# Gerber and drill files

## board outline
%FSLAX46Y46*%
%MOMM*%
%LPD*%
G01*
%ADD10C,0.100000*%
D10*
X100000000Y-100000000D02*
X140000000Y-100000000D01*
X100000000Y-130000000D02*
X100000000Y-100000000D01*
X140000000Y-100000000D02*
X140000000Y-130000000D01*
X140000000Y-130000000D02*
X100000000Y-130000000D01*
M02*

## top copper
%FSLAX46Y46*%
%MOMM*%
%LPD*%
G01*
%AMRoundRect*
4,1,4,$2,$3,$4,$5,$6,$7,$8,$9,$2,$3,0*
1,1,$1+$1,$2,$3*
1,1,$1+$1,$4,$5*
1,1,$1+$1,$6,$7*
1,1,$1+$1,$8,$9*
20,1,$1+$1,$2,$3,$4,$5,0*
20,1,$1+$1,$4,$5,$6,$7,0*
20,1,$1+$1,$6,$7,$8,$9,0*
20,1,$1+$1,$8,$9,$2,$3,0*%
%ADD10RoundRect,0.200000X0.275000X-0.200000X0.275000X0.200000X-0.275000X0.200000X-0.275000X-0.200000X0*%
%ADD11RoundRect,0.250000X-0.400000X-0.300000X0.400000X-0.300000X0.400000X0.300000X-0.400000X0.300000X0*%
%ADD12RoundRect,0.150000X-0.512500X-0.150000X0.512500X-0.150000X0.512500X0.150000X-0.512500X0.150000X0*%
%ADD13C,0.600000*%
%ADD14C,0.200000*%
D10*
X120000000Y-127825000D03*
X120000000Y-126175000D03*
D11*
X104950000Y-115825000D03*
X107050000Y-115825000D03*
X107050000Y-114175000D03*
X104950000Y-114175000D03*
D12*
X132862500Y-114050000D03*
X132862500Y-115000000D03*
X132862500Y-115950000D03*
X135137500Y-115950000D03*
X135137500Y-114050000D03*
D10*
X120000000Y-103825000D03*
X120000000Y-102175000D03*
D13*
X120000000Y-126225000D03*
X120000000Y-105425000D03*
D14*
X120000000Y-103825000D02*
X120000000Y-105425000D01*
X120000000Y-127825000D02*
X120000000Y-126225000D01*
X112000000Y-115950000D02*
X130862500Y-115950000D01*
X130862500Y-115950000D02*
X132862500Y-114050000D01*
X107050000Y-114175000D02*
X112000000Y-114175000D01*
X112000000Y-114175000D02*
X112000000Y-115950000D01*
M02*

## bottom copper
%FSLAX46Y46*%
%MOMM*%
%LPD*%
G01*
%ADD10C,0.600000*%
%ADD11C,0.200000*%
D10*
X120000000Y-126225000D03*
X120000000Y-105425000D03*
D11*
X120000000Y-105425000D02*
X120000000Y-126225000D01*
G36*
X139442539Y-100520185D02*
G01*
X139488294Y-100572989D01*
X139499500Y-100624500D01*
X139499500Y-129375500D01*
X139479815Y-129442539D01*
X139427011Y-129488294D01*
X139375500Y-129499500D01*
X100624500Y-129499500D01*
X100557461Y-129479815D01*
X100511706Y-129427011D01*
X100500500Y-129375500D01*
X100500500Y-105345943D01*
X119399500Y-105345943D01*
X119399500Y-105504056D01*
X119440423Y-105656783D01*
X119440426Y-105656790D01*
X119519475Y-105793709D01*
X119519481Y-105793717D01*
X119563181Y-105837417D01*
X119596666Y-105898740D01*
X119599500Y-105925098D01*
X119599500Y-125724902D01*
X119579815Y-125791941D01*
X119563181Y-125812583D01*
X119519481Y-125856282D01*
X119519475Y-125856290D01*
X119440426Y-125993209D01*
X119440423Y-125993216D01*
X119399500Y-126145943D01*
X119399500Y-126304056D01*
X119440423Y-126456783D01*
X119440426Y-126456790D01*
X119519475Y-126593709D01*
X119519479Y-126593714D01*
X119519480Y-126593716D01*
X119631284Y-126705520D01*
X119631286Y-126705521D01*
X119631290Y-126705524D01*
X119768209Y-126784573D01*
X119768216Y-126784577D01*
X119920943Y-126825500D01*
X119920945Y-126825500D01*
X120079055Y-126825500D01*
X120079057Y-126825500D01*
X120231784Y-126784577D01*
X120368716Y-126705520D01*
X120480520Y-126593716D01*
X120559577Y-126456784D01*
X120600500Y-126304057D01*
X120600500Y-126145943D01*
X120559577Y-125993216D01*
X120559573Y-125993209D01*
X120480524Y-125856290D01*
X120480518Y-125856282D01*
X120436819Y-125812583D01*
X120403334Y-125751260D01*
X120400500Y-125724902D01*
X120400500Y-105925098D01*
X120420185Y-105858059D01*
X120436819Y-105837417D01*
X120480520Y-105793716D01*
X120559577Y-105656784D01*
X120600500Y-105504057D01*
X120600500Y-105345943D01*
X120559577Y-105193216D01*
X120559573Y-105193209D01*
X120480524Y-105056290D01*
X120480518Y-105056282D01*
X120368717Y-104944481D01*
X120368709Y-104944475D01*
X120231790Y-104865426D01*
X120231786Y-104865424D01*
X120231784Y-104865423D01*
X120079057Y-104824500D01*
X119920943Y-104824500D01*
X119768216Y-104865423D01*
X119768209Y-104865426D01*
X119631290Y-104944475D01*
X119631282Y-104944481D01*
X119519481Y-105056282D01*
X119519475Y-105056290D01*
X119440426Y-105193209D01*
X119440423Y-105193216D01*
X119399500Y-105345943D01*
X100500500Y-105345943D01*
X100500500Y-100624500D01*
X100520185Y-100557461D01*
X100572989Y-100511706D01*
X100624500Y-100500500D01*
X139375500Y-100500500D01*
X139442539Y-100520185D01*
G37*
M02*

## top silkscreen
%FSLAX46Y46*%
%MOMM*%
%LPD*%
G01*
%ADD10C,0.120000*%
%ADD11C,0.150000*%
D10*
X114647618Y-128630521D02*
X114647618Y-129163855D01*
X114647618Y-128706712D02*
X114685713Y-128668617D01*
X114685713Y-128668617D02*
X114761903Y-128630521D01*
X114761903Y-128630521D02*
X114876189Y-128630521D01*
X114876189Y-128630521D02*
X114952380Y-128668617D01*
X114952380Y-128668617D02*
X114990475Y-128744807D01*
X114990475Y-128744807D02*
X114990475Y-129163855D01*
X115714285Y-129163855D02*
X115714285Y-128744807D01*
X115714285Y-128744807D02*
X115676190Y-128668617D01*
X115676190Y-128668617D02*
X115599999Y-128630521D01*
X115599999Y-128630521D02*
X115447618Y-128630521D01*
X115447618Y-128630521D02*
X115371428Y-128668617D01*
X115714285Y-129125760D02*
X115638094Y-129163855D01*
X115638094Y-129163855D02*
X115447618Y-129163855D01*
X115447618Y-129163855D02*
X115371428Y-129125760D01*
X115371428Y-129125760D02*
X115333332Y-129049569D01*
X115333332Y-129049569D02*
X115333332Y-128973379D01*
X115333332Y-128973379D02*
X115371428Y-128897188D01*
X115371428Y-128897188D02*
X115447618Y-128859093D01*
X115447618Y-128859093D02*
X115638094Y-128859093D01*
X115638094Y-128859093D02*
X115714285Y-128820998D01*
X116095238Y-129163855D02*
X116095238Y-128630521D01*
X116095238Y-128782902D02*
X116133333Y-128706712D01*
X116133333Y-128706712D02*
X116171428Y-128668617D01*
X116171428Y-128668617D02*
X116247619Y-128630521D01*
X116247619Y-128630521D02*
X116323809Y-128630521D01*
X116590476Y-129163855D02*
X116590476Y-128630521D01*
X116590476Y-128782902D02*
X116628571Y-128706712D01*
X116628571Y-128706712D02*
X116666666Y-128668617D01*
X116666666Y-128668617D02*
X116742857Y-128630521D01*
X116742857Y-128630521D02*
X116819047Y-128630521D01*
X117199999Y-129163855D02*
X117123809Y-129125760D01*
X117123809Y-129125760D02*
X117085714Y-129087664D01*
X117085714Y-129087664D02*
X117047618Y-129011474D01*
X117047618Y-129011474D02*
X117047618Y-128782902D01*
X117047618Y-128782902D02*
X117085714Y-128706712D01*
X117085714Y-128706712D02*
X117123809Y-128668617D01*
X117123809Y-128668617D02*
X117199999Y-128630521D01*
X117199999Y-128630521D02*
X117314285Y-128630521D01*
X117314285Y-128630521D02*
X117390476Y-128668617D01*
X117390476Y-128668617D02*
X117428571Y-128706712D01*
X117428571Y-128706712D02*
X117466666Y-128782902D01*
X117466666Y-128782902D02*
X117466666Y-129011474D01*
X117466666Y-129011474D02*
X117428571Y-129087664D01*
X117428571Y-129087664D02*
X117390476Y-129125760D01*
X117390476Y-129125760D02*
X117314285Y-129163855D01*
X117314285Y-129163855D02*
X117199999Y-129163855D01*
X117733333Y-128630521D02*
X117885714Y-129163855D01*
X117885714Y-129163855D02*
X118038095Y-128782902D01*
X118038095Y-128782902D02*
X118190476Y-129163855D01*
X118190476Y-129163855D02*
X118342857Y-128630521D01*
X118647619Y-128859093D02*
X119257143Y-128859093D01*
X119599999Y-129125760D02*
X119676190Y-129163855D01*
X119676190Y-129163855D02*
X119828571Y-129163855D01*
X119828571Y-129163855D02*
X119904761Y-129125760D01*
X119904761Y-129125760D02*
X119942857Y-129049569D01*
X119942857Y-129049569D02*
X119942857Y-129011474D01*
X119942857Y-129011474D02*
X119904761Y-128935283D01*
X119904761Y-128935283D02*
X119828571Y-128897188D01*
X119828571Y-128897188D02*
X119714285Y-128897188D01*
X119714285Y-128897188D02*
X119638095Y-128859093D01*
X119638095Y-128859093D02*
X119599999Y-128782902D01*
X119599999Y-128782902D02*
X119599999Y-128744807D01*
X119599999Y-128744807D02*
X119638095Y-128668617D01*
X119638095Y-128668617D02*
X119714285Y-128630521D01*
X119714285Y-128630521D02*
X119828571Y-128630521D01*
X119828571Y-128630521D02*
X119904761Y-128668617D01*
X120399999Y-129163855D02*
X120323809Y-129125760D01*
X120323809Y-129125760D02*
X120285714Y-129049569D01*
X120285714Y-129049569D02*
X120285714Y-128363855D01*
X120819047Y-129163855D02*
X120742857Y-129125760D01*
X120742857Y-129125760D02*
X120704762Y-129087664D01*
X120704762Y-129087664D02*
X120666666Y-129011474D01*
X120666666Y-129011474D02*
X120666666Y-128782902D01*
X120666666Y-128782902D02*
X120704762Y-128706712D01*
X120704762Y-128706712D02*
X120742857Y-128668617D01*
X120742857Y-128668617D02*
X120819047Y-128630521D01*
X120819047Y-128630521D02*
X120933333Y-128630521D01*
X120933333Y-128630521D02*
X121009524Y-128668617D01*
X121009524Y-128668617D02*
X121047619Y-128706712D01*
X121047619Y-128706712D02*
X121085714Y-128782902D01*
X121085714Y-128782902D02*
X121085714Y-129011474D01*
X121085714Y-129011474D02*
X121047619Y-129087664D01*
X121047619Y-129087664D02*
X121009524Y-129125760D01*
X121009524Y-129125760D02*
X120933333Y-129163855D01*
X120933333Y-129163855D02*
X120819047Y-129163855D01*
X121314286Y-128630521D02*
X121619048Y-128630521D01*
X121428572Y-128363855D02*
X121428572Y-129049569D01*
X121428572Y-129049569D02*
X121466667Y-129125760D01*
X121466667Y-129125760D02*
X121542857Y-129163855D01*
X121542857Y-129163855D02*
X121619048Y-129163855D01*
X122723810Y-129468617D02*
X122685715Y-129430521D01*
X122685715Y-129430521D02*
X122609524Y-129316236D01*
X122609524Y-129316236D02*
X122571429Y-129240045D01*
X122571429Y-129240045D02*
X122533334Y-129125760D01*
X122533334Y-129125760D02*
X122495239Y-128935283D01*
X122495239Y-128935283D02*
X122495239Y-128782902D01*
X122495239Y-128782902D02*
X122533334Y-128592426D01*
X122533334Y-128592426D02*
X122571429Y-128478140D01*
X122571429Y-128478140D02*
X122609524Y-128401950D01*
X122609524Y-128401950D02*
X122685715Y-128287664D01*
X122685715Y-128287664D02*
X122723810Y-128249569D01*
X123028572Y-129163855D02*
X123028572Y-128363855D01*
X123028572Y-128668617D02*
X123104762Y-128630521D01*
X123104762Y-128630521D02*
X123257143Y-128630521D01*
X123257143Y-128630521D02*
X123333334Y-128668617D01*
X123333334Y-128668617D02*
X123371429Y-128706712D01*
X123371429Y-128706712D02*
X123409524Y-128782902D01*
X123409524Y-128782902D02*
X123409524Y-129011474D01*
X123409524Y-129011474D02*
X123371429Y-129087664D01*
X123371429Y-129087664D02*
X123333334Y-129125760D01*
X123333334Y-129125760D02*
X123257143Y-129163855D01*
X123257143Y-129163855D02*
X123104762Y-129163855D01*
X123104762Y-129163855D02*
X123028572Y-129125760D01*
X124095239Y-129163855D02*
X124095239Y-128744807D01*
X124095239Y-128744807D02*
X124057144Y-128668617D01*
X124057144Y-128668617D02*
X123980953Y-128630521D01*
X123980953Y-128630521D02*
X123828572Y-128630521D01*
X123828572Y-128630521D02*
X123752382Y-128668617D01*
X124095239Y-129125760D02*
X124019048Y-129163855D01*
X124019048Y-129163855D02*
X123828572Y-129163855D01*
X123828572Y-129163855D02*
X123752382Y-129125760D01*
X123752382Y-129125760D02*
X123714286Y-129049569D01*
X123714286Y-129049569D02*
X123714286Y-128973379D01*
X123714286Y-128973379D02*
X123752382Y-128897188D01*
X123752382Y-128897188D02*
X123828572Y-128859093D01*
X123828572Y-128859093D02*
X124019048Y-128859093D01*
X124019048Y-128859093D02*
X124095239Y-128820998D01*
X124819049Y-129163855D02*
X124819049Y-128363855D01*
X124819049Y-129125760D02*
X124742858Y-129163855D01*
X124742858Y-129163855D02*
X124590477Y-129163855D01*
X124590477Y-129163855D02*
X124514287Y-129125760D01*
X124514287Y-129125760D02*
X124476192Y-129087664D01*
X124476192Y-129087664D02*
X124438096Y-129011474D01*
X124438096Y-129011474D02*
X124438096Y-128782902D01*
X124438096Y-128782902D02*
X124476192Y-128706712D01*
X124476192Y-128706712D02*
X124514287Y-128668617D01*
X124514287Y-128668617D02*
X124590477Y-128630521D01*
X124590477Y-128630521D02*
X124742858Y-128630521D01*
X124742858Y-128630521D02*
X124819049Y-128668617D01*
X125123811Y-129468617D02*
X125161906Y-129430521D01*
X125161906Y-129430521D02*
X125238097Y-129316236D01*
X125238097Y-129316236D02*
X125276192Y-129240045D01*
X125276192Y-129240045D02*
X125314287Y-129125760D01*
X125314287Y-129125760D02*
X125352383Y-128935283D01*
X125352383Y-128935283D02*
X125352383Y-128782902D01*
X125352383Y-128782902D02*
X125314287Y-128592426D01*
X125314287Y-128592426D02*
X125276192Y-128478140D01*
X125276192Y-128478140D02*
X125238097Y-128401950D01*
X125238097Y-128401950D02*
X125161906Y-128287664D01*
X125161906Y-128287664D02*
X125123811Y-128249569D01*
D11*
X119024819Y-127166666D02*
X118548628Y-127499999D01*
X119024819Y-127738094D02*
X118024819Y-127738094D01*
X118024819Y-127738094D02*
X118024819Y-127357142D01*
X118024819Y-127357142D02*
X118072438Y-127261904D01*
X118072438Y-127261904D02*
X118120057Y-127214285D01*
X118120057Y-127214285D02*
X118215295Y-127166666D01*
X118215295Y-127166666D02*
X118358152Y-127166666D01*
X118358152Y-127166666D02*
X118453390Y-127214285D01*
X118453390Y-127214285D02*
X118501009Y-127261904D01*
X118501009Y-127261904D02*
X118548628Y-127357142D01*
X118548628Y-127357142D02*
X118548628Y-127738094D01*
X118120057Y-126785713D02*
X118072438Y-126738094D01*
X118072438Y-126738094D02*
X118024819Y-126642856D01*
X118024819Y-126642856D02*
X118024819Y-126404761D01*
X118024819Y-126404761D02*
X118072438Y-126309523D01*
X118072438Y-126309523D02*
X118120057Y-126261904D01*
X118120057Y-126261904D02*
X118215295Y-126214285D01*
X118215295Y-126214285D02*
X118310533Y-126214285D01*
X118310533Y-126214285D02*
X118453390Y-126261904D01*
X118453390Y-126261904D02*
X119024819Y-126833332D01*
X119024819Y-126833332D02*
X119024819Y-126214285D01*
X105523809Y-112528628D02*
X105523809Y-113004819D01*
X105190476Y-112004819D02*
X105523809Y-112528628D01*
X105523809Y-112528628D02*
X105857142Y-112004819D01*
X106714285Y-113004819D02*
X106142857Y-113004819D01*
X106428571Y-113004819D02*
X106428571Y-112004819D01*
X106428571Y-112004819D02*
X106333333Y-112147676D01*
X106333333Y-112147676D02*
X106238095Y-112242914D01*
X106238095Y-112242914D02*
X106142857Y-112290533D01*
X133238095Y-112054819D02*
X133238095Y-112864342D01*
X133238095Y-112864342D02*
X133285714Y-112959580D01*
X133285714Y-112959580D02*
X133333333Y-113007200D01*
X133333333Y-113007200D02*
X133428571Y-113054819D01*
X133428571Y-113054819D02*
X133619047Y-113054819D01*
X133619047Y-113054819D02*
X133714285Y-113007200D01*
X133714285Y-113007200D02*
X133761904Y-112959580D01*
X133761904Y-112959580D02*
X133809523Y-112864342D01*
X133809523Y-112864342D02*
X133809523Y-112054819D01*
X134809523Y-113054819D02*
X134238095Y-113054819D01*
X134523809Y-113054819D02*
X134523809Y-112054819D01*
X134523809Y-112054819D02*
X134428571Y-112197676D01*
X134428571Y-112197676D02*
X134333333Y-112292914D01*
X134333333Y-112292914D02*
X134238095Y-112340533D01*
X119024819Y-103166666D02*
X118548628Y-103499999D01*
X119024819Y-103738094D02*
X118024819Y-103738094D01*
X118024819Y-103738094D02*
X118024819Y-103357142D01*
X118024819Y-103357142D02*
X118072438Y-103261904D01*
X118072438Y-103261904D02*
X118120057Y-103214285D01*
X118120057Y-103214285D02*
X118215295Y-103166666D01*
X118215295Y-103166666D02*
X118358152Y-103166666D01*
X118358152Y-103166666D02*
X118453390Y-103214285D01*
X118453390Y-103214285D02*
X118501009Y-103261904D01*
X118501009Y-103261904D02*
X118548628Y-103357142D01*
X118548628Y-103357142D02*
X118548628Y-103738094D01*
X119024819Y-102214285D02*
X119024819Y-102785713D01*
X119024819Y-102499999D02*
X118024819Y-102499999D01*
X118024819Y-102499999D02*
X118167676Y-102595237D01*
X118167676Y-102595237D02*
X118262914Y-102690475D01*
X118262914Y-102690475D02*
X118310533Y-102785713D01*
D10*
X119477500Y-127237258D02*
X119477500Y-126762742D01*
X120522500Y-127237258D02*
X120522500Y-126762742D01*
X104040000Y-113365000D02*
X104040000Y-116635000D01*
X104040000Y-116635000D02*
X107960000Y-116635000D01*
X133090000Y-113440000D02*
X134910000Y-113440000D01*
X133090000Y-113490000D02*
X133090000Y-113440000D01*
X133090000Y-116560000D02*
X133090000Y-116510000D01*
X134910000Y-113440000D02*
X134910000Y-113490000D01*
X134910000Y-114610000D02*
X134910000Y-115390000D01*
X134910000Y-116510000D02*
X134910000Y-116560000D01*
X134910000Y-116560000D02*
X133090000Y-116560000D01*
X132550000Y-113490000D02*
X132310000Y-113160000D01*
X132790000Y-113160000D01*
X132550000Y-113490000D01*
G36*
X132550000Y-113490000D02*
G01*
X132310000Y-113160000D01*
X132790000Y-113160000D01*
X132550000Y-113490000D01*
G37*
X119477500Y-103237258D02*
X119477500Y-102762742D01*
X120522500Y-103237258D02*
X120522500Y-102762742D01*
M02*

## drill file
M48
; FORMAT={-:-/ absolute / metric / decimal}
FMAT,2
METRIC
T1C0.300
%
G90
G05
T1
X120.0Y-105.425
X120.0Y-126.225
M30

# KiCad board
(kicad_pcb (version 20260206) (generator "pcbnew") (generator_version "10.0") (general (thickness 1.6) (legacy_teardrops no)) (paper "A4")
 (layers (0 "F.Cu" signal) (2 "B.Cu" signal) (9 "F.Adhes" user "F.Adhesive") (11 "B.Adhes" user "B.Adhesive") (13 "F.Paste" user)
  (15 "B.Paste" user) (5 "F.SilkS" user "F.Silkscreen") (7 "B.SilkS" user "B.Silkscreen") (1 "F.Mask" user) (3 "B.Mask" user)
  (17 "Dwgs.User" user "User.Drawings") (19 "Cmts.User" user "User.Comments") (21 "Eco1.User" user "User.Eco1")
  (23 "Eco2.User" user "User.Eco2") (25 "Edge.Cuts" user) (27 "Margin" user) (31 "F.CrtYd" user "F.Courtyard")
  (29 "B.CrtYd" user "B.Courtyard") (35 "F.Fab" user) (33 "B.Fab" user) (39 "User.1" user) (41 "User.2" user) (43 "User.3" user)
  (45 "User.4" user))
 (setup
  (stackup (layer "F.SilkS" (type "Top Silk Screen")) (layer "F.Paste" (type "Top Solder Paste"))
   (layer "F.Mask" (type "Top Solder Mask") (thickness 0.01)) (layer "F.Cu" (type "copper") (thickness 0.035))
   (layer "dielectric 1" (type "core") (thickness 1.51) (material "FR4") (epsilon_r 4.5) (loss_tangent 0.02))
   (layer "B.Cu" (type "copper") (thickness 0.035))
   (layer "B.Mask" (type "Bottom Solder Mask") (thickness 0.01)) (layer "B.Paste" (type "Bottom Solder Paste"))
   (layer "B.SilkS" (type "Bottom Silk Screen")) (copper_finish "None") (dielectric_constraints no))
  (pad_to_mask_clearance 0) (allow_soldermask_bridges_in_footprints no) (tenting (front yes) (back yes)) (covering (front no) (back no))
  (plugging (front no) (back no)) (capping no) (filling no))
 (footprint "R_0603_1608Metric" (layer "F.Cu") (at 120 127 90)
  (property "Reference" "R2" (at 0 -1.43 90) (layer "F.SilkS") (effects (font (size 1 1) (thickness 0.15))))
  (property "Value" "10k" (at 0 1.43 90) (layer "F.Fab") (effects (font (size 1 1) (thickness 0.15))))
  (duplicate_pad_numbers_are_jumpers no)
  (fp_line (start -0.237258 -0.5225) (end 0.237258 -0.5225) (stroke (width 0.12) (type solid)) (layer "F.SilkS"))
  (fp_line (start -0.237258 0.5225) (end 0.237258 0.5225) (stroke (width 0.12) (type solid)) (layer "F.SilkS"))
  (pad "1" smd roundrect (at -0.825 0 90) (size 0.8 0.95) (layers "F.Cu" "F.Mask" "F.Paste") (roundrect_rratio 0.25) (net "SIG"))
  (pad "2" smd roundrect (at 0.825 0 90) (size 0.8 0.95) (layers "F.Cu" "F.Mask" "F.Paste") (roundrect_rratio 0.25) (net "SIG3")))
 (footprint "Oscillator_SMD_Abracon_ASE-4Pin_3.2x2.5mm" (layer "F.Cu") (at 106 115)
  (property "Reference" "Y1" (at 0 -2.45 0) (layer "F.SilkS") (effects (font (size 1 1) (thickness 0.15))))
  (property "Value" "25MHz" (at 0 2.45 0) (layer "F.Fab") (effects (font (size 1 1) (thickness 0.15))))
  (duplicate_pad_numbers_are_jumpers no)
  (fp_line (start -1.96 -1.635) (end -1.96 1.635) (stroke (width 0.12) (type solid)) (layer "F.SilkS"))
  (fp_line (start -1.96 1.635) (end 1.96 1.635) (stroke (width 0.12) (type solid)) (layer "F.SilkS"))
  (pad "1" smd roundrect (at -1.05 0.825) (size 1.3 1.1) (layers "F.Cu" "F.Mask" "F.Paste") (roundrect_rratio 0.227273) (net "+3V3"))
  (pad "2" smd roundrect (at 1.05 0.825) (size 1.3 1.1) (layers "F.Cu" "F.Mask" "F.Paste") (roundrect_rratio 0.227273) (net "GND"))
  (pad "3" smd roundrect (at 1.05 -0.825) (size 1.3 1.1) (layers "F.Cu" "F.Mask" "F.Paste") (roundrect_rratio 0.227273) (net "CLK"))
  (pad "4" smd roundrect (at -1.05 -0.825) (size 1.3 1.1) (layers "F.Cu" "F.Mask" "F.Paste") (roundrect_rratio 0.227273) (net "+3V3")))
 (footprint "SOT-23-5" (layer "F.Cu") (at 134 115)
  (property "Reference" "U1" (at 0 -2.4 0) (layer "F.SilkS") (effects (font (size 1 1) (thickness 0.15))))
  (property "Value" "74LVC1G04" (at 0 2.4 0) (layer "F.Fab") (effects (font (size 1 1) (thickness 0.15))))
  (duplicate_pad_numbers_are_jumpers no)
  (fp_line (start -0.91 -1.56) (end 0.91 -1.56) (stroke (width 0.12) (type solid)) (layer "F.SilkS"))
  (fp_line (start -0.91 -1.51) (end -0.91 -1.56) (stroke (width 0.12) (type solid)) (layer "F.SilkS"))
  (fp_line (start -0.91 1.56) (end -0.91 1.51) (stroke (width 0.12) (type solid)) (layer "F.SilkS"))
  (fp_line (start 0.91 -1.56) (end 0.91 -1.51) (stroke (width 0.12) (type solid)) (layer "F.SilkS"))
  (fp_line (start 0.91 -0.39) (end 0.91 0.39) (stroke (width 0.12) (type solid)) (layer "F.SilkS"))
  (fp_line (start 0.91 1.51) (end 0.91 1.56) (stroke (width 0.12) (type solid)) (layer "F.SilkS"))
  (fp_line (start 0.91 1.56) (end -0.91 1.56) (stroke (width 0.12) (type solid)) (layer "F.SilkS"))
  (fp_poly (pts (xy -1.45 -1.51) (xy -1.69 -1.84) (xy -1.21 -1.84)) (stroke (width 0.12) (type solid)) (fill yes) (layer "F.SilkS"))
  (pad "1" smd roundrect (at -1.1375 -0.95) (size 1.325 0.6) (layers "F.Cu" "F.Mask" "F.Paste") (roundrect_rratio 0.25) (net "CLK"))
  (pad "2" smd roundrect (at -1.1375 0) (size 1.325 0.6) (layers "F.Cu" "F.Mask" "F.Paste") (roundrect_rratio 0.25) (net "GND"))
  (pad "3" smd roundrect (at -1.1375 0.95) (size 1.325 0.6) (layers "F.Cu" "F.Mask" "F.Paste") (roundrect_rratio 0.25))
  (pad "4" smd roundrect (at 1.1375 0.95) (size 1.325 0.6) (layers "F.Cu" "F.Mask" "F.Paste") (roundrect_rratio 0.25))
  (pad "5" smd roundrect (at 1.1375 -0.95) (size 1.325 0.6) (layers "F.Cu" "F.Mask" "F.Paste") (roundrect_rratio 0.25) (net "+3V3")))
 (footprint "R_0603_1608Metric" (layer "F.Cu") (at 120 103 90)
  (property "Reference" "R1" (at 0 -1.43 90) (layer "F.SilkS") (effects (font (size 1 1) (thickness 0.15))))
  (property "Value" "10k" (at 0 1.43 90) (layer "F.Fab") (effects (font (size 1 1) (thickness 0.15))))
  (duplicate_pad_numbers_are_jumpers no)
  (fp_line (start -0.237258 -0.5225) (end 0.237258 -0.5225) (stroke (width 0.12) (type solid)) (layer "F.SilkS"))
  (fp_line (start -0.237258 0.5225) (end 0.237258 0.5225) (stroke (width 0.12) (type solid)) (layer "F.SilkS"))
  (pad "1" smd roundrect (at -0.825 0 90) (size 0.8 0.95) (layers "F.Cu" "F.Mask" "F.Paste") (roundrect_rratio 0.25) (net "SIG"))
  (pad "2" smd roundrect (at 0.825 0 90) (size 0.8 0.95) (layers "F.Cu" "F.Mask" "F.Paste") (roundrect_rratio 0.25) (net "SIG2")))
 (gr_line (start 100 100) (end 140 100) (stroke (width 0.1) (type default)) (layer "Edge.Cuts"))
 (gr_line (start 100 130) (end 100 100) (stroke (width 0.1) (type default)) (layer "Edge.Cuts"))
 (gr_line (start 140 100) (end 140 130) (stroke (width 0.1) (type default)) (layer "Edge.Cuts"))
 (gr_line (start 140 130) (end 100 130) (stroke (width 0.1) (type default)) (layer "Edge.Cuts"))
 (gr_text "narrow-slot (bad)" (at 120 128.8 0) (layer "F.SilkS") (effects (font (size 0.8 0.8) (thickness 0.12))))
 (segment (start 120 103.825) (end 120 105.425) (width 0.2) (layer "F.Cu") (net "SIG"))
 (segment (start 120 127.825) (end 120 126.225) (width 0.2) (layer "F.Cu") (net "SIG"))
 (via (at 120 126.225) (size 0.6) (drill 0.3) (layers "F.Cu" "B.Cu") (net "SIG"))
 (via (at 120 105.425) (size 0.6) (drill 0.3) (layers "F.Cu" "B.Cu") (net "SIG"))
 (segment (start 120 105.425) (end 120 126.225) (width 0.2) (layer "B.Cu") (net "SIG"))
 (segment (start 112 115.95) (end 130.8625 115.95) (width 0.2) (layer "F.Cu") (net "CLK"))
 (segment (start 130.8625 115.95) (end 132.8625 114.05) (width 0.2) (layer "F.Cu") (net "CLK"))
 (segment (start 107.05 114.175) (end 112 114.175) (width 0.2) (layer "F.Cu") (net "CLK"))
 (segment (start 112 114.175) (end 112 115.95) (width 0.2) (layer "F.Cu") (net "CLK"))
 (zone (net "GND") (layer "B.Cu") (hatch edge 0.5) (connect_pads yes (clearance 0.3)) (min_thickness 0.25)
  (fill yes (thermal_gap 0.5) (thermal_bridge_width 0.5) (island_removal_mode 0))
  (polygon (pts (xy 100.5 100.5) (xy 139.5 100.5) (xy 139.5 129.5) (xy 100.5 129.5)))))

